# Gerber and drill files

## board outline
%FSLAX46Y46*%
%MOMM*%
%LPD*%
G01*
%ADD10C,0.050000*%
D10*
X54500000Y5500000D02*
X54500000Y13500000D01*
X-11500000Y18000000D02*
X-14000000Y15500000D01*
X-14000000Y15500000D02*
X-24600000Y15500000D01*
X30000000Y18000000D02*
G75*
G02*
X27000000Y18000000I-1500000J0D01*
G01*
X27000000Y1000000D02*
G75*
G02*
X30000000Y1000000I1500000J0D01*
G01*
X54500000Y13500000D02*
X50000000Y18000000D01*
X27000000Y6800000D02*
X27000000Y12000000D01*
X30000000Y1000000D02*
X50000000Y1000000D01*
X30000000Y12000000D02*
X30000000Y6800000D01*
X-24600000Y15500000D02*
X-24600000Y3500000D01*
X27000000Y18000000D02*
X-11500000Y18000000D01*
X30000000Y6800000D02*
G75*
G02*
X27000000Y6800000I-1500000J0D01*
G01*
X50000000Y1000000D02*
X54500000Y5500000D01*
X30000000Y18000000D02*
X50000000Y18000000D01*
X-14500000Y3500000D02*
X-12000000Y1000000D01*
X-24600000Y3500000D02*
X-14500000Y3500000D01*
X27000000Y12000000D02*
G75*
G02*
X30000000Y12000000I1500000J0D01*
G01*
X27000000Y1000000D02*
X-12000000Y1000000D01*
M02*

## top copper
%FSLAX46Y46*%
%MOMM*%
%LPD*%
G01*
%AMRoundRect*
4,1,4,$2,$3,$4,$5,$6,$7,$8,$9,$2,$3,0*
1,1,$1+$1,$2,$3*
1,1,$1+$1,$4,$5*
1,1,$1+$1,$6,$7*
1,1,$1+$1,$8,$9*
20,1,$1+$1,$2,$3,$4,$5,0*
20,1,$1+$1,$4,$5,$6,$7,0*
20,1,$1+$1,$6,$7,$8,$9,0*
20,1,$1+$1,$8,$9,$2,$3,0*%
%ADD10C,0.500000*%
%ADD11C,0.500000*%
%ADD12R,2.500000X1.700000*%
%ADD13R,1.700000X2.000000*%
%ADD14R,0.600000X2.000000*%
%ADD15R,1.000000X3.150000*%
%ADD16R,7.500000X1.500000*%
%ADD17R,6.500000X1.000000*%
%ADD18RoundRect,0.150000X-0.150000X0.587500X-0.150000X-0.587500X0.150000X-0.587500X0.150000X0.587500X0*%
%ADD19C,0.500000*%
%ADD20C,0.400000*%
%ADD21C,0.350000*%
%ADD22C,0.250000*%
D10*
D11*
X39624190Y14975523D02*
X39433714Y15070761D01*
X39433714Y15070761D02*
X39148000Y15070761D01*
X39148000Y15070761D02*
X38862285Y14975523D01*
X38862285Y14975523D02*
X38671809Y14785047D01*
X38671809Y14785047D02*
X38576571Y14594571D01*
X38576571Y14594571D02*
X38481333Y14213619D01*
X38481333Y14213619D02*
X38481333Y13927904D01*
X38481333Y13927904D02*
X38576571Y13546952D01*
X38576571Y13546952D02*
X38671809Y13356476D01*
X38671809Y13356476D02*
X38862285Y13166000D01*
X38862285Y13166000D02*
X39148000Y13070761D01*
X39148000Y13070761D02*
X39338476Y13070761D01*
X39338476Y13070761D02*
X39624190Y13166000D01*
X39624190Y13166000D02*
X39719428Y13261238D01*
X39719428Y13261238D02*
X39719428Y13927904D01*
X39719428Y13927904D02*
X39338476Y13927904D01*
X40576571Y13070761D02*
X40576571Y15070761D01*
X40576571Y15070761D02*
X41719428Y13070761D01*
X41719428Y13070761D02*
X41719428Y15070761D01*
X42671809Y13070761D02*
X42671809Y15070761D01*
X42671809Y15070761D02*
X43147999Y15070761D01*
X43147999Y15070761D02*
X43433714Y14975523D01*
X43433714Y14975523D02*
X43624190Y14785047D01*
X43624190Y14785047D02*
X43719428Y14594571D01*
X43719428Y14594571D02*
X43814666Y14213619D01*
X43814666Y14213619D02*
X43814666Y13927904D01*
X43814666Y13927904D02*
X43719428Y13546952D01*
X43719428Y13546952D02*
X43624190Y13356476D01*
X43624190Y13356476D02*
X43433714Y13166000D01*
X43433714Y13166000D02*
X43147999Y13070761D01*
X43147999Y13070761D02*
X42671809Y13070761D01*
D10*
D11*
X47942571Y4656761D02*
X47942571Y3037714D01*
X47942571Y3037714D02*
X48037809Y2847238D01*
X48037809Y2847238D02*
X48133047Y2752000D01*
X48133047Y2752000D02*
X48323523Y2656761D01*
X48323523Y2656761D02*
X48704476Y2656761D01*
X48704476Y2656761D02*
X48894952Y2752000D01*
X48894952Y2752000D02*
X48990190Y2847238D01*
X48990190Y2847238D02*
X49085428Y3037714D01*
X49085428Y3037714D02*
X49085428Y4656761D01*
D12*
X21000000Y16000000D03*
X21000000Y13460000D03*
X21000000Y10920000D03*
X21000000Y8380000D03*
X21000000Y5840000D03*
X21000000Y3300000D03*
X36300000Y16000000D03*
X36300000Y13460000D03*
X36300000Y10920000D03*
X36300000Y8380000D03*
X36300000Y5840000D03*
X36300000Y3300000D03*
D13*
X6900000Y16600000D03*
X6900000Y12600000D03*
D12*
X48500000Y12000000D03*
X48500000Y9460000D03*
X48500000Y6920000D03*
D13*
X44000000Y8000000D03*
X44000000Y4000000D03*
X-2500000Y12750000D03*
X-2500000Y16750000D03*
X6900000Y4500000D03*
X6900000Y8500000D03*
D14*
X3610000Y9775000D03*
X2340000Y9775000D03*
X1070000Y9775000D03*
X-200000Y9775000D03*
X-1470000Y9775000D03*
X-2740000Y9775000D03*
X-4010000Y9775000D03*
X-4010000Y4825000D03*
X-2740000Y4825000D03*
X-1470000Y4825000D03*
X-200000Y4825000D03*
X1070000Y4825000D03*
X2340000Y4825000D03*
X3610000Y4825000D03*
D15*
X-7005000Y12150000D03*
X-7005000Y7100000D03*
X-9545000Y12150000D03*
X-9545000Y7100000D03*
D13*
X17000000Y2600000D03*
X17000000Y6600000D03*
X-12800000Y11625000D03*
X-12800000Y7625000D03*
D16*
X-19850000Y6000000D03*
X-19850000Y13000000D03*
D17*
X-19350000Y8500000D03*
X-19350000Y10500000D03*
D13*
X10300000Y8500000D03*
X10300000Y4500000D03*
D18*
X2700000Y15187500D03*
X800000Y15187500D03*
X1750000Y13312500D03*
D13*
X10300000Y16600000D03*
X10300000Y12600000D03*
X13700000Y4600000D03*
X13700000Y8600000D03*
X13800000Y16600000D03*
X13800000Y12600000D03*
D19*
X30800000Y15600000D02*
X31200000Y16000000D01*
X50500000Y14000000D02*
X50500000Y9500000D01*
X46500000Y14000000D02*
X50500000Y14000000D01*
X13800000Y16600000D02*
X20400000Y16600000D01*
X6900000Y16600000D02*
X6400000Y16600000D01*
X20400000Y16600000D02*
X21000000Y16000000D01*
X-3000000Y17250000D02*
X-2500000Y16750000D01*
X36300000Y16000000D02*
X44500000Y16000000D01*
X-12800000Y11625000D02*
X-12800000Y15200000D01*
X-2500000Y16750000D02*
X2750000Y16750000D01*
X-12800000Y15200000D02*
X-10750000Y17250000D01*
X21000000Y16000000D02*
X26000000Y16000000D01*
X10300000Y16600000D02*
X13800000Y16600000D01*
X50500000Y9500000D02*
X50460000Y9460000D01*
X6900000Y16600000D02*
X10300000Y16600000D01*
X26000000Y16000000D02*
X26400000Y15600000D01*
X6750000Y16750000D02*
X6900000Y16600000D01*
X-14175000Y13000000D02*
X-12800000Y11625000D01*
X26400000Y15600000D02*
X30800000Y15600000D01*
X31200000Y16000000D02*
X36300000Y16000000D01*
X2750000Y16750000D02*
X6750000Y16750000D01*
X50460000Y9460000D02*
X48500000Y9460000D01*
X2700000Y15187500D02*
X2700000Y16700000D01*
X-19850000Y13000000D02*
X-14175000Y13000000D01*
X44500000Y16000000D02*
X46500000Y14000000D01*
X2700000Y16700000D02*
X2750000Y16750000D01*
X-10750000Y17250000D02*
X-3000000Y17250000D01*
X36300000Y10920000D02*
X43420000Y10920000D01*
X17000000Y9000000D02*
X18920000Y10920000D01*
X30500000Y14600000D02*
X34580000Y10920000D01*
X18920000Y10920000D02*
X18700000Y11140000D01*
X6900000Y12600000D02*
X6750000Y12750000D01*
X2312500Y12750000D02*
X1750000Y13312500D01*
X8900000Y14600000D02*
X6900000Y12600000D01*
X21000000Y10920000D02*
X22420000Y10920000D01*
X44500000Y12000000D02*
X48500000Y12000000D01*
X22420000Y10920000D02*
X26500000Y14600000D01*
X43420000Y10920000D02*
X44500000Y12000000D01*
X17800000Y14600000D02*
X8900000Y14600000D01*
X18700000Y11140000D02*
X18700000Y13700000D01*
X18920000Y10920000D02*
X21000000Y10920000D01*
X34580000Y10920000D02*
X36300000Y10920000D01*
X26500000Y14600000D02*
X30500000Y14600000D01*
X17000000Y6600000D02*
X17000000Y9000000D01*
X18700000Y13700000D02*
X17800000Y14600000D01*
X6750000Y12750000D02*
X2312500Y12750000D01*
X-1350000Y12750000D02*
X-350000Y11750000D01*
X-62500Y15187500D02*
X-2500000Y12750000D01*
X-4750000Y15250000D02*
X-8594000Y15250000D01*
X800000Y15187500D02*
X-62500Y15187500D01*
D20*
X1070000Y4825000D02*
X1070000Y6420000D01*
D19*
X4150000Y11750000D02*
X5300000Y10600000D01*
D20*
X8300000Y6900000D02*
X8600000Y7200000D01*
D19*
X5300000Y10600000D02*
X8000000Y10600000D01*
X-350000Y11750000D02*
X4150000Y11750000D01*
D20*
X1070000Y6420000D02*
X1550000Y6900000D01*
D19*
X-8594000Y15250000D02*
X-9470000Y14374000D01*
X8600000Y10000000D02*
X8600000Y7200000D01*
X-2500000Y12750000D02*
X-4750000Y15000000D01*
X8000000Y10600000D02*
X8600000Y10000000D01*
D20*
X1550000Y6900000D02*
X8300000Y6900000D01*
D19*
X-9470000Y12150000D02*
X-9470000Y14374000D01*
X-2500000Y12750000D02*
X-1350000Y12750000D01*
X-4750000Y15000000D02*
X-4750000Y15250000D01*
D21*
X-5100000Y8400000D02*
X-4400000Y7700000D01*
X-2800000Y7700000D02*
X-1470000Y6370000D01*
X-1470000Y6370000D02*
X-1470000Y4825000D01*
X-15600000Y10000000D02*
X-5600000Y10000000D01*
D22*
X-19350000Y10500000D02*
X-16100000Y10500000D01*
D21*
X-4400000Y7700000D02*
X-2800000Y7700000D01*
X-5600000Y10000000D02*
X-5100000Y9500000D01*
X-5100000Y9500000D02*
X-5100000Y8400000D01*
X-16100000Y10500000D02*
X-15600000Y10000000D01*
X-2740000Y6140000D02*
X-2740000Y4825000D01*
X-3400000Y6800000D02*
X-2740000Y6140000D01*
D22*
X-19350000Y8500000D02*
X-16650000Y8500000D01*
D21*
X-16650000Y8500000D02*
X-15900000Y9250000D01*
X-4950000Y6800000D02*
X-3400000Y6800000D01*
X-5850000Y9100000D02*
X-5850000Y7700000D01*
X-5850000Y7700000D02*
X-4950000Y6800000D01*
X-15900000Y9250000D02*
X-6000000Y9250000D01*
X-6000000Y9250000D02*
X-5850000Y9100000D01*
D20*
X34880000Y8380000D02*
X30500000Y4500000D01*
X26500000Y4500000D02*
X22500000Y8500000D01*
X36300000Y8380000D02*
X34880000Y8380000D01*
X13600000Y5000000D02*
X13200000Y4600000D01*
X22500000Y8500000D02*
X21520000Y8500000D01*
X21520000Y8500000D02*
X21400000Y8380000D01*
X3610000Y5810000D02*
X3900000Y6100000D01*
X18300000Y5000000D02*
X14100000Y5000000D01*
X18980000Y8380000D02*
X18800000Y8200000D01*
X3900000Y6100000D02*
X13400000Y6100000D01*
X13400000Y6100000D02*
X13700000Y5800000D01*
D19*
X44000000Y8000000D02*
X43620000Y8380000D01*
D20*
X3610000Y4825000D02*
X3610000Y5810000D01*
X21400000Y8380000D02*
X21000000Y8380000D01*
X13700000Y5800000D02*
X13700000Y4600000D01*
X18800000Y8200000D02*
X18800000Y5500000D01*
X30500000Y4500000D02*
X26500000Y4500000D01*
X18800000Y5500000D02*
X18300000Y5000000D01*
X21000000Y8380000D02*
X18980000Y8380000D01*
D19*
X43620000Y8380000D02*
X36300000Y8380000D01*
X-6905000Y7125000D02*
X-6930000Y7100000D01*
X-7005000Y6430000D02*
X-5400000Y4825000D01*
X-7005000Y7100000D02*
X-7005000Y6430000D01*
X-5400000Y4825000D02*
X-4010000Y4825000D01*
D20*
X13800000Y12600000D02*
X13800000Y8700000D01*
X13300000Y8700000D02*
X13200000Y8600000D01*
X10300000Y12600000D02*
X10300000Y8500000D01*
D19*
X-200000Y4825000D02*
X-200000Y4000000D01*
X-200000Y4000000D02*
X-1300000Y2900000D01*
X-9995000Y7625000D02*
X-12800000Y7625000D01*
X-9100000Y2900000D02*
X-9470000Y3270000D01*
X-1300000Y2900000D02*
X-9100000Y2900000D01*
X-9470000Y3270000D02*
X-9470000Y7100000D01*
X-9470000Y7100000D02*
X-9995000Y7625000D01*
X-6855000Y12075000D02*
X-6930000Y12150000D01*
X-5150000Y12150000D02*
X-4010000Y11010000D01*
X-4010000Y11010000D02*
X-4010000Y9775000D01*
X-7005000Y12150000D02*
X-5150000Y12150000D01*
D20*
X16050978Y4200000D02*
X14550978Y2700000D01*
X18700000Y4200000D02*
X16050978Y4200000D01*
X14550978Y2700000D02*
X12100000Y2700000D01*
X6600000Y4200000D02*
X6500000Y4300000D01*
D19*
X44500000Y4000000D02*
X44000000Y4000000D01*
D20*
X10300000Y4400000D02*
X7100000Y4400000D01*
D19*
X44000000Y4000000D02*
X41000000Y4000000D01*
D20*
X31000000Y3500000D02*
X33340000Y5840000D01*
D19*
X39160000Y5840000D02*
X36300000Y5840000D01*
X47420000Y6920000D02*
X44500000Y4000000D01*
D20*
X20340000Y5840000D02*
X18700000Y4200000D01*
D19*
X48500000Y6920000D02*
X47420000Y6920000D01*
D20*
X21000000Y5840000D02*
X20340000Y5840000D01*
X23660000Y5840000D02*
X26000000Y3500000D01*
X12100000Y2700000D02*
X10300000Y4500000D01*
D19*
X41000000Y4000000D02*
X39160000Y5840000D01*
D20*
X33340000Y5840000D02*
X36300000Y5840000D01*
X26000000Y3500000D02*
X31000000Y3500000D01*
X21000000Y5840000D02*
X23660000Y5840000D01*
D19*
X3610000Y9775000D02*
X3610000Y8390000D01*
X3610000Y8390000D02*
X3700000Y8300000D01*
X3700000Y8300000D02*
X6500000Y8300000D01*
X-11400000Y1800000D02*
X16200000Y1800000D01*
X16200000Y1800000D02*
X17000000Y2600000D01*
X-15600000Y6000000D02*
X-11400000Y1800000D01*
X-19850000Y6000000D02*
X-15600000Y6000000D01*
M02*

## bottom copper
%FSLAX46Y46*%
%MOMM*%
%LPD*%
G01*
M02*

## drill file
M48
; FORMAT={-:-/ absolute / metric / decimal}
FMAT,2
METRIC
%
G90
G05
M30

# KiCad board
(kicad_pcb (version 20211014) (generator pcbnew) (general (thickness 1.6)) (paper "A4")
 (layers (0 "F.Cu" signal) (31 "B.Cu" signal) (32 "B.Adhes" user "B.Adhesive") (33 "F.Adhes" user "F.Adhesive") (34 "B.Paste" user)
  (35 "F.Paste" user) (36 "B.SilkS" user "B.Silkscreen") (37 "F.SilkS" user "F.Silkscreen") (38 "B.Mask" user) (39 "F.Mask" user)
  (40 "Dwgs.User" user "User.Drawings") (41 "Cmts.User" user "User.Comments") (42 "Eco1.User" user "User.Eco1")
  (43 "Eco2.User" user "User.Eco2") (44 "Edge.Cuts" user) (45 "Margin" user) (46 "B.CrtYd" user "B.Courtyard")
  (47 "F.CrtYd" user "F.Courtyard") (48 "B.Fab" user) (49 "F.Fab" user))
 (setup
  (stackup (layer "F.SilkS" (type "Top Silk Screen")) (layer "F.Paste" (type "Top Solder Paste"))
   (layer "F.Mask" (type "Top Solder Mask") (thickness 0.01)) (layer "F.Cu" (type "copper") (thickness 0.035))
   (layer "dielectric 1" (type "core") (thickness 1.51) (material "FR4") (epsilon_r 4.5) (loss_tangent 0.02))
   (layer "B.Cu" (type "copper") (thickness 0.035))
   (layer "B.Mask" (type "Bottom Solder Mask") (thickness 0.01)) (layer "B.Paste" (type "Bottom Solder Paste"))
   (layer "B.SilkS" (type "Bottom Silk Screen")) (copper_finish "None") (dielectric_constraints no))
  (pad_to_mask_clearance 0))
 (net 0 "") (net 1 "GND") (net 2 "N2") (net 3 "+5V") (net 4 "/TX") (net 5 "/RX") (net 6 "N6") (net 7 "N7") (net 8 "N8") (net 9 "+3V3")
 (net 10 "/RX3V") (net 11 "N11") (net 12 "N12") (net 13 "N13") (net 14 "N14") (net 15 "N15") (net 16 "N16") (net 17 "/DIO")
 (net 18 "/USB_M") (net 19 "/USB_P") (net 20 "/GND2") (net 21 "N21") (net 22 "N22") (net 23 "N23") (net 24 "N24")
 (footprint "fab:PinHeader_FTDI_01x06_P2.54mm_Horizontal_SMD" (layer "F.Cu") (at 21 -16)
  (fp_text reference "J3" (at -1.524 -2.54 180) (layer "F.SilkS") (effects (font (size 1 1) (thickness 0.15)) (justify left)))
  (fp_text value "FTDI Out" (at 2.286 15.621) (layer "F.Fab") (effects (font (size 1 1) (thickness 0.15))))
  (pad "1" smd rect locked (at 0 0) (size 2.5 1.7) (layers "F.Cu" "F.Paste" "F.Mask") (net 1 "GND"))
  (pad "2" smd rect locked (at 0 2.54) (size 2.5 1.7) (layers "F.Cu" "F.Paste" "F.Mask") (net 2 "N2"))
  (pad "3" smd rect locked (at 0 5.08) (size 2.5 1.7) (layers "F.Cu" "F.Paste" "F.Mask") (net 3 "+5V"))
  (pad "4" smd rect locked (at 0 7.62) (size 2.5 1.7) (layers "F.Cu" "F.Paste" "F.Mask") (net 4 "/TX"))
  (pad "5" smd rect locked (at 0 10.16) (size 2.5 1.7) (layers "F.Cu" "F.Paste" "F.Mask") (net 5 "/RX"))
  (pad "6" smd rect locked (at 0 12.7) (size 2.5 1.7) (layers "F.Cu" "F.Paste" "F.Mask") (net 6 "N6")))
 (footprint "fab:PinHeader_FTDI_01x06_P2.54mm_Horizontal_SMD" (layer "F.Cu") (at 36.3 -16)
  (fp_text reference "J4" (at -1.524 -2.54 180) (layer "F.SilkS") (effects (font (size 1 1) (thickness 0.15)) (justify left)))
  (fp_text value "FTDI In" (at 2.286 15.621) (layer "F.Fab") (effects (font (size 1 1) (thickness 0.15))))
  (pad "1" smd rect locked (at 0 0) (size 2.5 1.7) (layers "F.Cu" "F.Paste" "F.Mask") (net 1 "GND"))
  (pad "2" smd rect locked (at 0 2.54) (size 2.5 1.7) (layers "F.Cu" "F.Paste" "F.Mask") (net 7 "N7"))
  (pad "3" smd rect locked (at 0 5.08) (size 2.5 1.7) (layers "F.Cu" "F.Paste" "F.Mask") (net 3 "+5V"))
  (pad "4" smd rect locked (at 0 7.62) (size 2.5 1.7) (layers "F.Cu" "F.Paste" "F.Mask") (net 4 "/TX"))
  (pad "5" smd rect locked (at 0 10.16) (size 2.5 1.7) (layers "F.Cu" "F.Paste" "F.Mask") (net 5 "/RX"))
  (pad "6" smd rect locked (at 0 12.7) (size 2.5 1.7) (layers "F.Cu" "F.Paste" "F.Mask") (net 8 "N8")))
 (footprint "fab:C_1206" (layer "F.Cu") (at 6.9 -14.6 -90)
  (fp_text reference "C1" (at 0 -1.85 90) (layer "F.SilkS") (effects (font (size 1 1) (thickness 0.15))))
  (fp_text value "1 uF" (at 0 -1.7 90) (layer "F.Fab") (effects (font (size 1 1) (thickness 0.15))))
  (pad "1" smd rect locked (at -2 0 270) (size 2 1.7) (layers "F.Cu" "F.Paste" "F.Mask") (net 1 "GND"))
  (pad "2" smd rect locked (at 2 0 270) (size 2 1.7) (layers "F.Cu" "F.Paste" "F.Mask") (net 3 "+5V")))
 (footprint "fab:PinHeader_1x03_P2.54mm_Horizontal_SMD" (layer "F.Cu") (at 48.5 -12)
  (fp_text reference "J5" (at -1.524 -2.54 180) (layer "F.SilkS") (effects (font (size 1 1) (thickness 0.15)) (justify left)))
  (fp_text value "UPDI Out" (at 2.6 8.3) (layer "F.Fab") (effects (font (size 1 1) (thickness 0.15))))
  (pad "1" smd rect locked (at 0 0) (size 2.5 1.7) (layers "F.Cu" "F.Paste" "F.Mask") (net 3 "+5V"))
  (pad "2" smd rect locked (at 0 2.54) (size 2.5 1.7) (layers "F.Cu" "F.Paste" "F.Mask") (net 1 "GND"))
  (pad "3" smd rect locked (at 0 5.08) (size 2.5 1.7) (layers "F.Cu" "F.Paste" "F.Mask") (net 5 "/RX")))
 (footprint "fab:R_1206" (layer "F.Cu") (at 44 -6 -90)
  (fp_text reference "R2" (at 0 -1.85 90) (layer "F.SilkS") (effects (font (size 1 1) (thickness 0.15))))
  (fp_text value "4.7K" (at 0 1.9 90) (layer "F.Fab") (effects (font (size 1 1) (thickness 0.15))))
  (pad "1" smd rect locked (at -2 0 270) (size 2 1.7) (layers "F.Cu" "F.Paste" "F.Mask") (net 4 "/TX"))
  (pad "2" smd rect locked (at 2 0 270) (size 2 1.7) (layers "F.Cu" "F.Paste" "F.Mask") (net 5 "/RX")))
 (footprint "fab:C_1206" (layer "F.Cu") (at -2.5 -14.75 90)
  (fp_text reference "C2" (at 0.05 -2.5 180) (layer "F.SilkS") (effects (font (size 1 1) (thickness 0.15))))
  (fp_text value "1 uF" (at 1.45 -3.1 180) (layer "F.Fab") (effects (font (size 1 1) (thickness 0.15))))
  (pad "1" smd rect locked (at -2 0 90) (size 2 1.7) (layers "F.Cu" "F.Paste" "F.Mask") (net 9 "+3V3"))
  (pad "2" smd rect locked (at 2 0 90) (size 2 1.7) (layers "F.Cu" "F.Paste" "F.Mask") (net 1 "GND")))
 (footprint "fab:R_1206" (layer "F.Cu") (at 6.9 -6.5 90)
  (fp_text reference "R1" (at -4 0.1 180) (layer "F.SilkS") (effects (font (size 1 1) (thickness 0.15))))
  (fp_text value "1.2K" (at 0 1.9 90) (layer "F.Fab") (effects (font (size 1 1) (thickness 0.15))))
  (pad "1" smd rect locked (at -2 0 90) (size 2 1.7) (layers "F.Cu" "F.Paste" "F.Mask") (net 5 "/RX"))
  (pad "2" smd rect locked (at 2 0 90) (size 2 1.7) (layers "F.Cu" "F.Paste" "F.Mask") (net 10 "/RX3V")))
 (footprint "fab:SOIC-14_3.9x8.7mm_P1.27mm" (layer "F.Cu") (at -0.2 -7.3 -90)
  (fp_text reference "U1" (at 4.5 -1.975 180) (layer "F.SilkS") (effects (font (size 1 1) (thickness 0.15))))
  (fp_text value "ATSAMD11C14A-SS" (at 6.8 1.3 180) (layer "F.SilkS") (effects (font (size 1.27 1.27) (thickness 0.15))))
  (pad "1" smd rect locked (at -2.475 -3.81 270) (size 2 0.6) (layers "F.Cu" "F.Paste" "F.Mask") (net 10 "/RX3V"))
  (pad "2" smd rect locked (at -2.475 -2.54 270) (size 2 0.6) (layers "F.Cu" "F.Paste" "F.Mask") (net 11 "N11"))
  (pad "3" smd rect locked (at -2.475 -1.27 270) (size 2 0.6) (layers "F.Cu" "F.Paste" "F.Mask") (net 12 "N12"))
  (pad "4" smd rect locked (at -2.475 0 270) (size 2 0.6) (layers "F.Cu" "F.Paste" "F.Mask") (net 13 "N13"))
  (pad "5" smd rect locked (at -2.475 1.27 270) (size 2 0.6) (layers "F.Cu" "F.Paste" "F.Mask") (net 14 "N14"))
  (pad "6" smd rect locked (at -2.475 2.54 270) (size 2 0.6) (layers "F.Cu" "F.Paste" "F.Mask") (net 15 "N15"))
  (pad "7" smd rect locked (at -2.475 3.81 270) (size 2 0.6) (layers "F.Cu" "F.Paste" "F.Mask") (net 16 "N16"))
  (pad "8" smd rect locked (at 2.475 3.81 270) (size 2 0.6) (layers "F.Cu" "F.Paste" "F.Mask") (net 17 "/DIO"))
  (pad "9" smd rect locked (at 2.475 2.54 270) (size 2 0.6) (layers "F.Cu" "F.Paste" "F.Mask") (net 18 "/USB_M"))
  (pad "10" smd rect locked (at 2.475 1.27 270) (size 2 0.6) (layers "F.Cu" "F.Paste" "F.Mask") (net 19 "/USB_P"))
  (pad "11" smd rect locked (at 2.475 0 270) (size 2 0.6) (layers "F.Cu" "F.Paste" "F.Mask") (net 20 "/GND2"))
  (pad "12" smd rect locked (at 2.475 -1.27 270) (size 2 0.6) (layers "F.Cu" "F.Paste" "F.Mask") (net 9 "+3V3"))
  (pad "13" smd rect locked (at 2.475 -2.54 270) (size 2 0.6) (layers "F.Cu" "F.Paste" "F.Mask") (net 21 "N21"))
  (pad "14" smd rect locked (at 2.475 -3.81 270) (size 2 0.6) (layers "F.Cu" "F.Paste" "F.Mask") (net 4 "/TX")))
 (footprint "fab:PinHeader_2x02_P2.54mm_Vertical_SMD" (layer "F.Cu") (at -8.275 -9.625 -90)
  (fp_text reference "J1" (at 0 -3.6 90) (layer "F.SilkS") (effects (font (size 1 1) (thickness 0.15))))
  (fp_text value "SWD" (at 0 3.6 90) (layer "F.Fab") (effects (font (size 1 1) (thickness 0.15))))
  (pad "1" smd rect locked (at -2.525 -1.27 270) (size 3.15 1) (layers "F.Cu" "F.Paste" "F.Mask") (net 16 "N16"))
  (pad "2" smd rect locked (at 2.525 -1.27 270) (size 3.15 1) (layers "F.Cu" "F.Paste" "F.Mask") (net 17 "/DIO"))
  (pad "3" smd rect locked (at -2.525 1.27 270) (size 3.15 1) (layers "F.Cu" "F.Paste" "F.Mask") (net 9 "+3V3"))
  (pad "4" smd rect locked (at 2.525 1.27 270) (size 3.15 1) (layers "F.Cu" "F.Paste" "F.Mask") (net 20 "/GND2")))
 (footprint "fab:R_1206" (layer "F.Cu") (at 17 -4.6 90)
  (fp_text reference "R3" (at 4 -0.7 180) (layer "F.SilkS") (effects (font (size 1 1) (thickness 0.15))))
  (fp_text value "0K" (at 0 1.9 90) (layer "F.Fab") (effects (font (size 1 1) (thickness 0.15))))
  (pad "1" smd rect locked (at -2 0 90) (size 2 1.7) (layers "F.Cu" "F.Paste" "F.Mask") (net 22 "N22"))
  (pad "2" smd rect locked (at 2 0 90) (size 2 1.7) (layers "F.Cu" "F.Paste" "F.Mask") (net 3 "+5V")))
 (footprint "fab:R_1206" (layer "F.Cu") (at -12.8 -9.625 -90)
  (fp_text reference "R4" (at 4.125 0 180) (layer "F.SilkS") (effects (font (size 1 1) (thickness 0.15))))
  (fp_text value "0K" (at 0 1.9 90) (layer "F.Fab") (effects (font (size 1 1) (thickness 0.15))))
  (pad "1" smd rect locked (at -2 0 270) (size 2 1.7) (layers "F.Cu" "F.Paste" "F.Mask") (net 1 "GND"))
  (pad "2" smd rect locked (at 2 0 270) (size 2 1.7) (layers "F.Cu" "F.Paste" "F.Mask") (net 20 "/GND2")))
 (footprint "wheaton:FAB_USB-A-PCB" (layer "F.Cu") (at -19.65 -9.5)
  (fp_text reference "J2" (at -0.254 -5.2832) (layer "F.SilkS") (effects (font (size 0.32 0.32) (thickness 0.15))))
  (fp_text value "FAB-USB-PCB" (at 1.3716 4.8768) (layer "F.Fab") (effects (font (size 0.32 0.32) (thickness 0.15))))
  (pad "5V" smd rect locked (at -0.2 3.5) (size 7.5 1.5) (layers "F.Cu" "F.Paste" "F.Mask") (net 22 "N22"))
  (pad "GND" smd rect locked (at -0.2 -3.5) (size 7.5 1.5) (layers "F.Cu" "F.Paste" "F.Mask") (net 1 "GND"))
  (pad "USB_M" smd rect locked (at 0.3 1) (size 6.5 1) (layers "F.Cu" "F.Paste" "F.Mask") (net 18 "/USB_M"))
  (pad "USB_P" smd rect locked (at 0.3 -1) (size 6.5 1) (layers "F.Cu" "F.Paste" "F.Mask") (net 19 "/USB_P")))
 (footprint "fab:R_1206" (layer "F.Cu") (at 10.3 -6.5 -90)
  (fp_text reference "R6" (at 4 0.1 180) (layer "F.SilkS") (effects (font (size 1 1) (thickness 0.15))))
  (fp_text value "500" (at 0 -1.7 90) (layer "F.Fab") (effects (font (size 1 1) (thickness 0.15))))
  (pad "1" smd rect locked (at -2 0 270) (size 2 1.7) (layers "F.Cu" "F.Paste" "F.Mask") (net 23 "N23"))
  (pad "2" smd rect locked (at 2 0 270) (size 2 1.7) (layers "F.Cu" "F.Paste" "F.Mask") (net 5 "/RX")))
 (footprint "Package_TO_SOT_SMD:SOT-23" (layer "F.Cu") (at 1.75 -14.25 -90)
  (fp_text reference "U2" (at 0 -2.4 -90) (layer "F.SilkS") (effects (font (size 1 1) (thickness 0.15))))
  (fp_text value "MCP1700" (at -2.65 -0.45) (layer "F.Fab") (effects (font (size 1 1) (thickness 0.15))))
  (pad "1" smd roundrect (at -0.9375 -0.95 270) (size 1.475 0.6) (layers "F.Cu" "F.Paste" "F.Mask") (roundrect_rratio 0.25) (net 1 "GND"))
  (pad "2" smd roundrect (at -0.9375 0.95 270) (size 1.475 0.6) (layers "F.Cu" "F.Paste" "F.Mask") (roundrect_rratio 0.25) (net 9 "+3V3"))
  (pad "3" smd roundrect (at 0.9375 0 270) (size 1.475 0.6) (layers "F.Cu" "F.Paste" "F.Mask") (roundrect_rratio 0.25) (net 3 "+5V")))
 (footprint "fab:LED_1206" (layer "F.Cu") (at 10.3 -14.6 -90)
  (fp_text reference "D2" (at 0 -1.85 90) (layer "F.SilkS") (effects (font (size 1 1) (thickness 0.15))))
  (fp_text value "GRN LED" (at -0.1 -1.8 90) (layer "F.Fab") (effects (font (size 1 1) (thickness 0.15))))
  (pad "1" smd rect locked (at -2 0 270) (size 2 1.7) (layers "F.Cu" "F.Paste" "F.Mask") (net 1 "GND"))
  (pad "2" smd rect locked (at 2 0 270) (size 2 1.7) (layers "F.Cu" "F.Paste" "F.Mask") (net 23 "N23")))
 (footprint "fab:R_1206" (layer "F.Cu") (at 13.7 -6.6 90)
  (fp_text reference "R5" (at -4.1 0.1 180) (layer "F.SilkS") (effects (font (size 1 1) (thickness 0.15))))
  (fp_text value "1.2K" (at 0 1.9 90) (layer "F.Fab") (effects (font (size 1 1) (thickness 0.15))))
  (pad "1" smd rect locked (at -2 0 90) (size 2 1.7) (layers "F.Cu" "F.Paste" "F.Mask") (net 4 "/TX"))
  (pad "2" smd rect locked (at 2 0 90) (size 2 1.7) (layers "F.Cu" "F.Paste" "F.Mask") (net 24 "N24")))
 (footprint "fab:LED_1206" (layer "F.Cu") (at 13.8 -14.6 -90)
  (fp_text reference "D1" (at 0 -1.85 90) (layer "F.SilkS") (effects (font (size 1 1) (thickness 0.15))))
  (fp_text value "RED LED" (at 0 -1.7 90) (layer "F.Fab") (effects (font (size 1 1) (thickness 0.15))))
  (pad "1" smd rect locked (at -2 0 270) (size 2 1.7) (layers "F.Cu" "F.Paste" "F.Mask") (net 1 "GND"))
  (pad "2" smd rect locked (at 2 0 270) (size 2 1.7) (layers "F.Cu" "F.Paste" "F.Mask") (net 24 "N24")))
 (gr_line (start 54.5 -5.5) (end 54.5 -13.5) (layer "Edge.Cuts") (width 0.05))
 (gr_line (start -11.5 -18) (end -14 -15.5) (layer "Edge.Cuts") (width 0.05))
 (gr_line (start -14 -15.5) (end -24.6 -15.5) (layer "Edge.Cuts") (width 0.05))
 (gr_arc (start 30 -18) (mid 28.5 -16.5) (end 27 -18) (layer "Edge.Cuts") (width 0.05))
 (gr_arc (start 27 -1) (mid 28.5 -2.5) (end 30 -1) (layer "Edge.Cuts") (width 0.05))
 (gr_line (start 54.5 -13.5) (end 50 -18) (layer "Edge.Cuts") (width 0.05))
 (gr_line (start 27 -6.8) (end 27 -12) (layer "Edge.Cuts") (width 0.05))
 (gr_line (start 30 -1) (end 50 -1) (layer "Edge.Cuts") (width 0.05))
 (gr_line (start 30 -12) (end 30 -6.8) (layer "Edge.Cuts") (width 0.05))
 (gr_line (start -24.6 -15.5) (end -24.6 -3.5) (layer "Edge.Cuts") (width 0.05))
 (gr_line (start 27 -18) (end -11.5 -18) (layer "Edge.Cuts") (width 0.05))
 (gr_arc (start 30 -6.8) (mid 28.5 -5.3) (end 27 -6.8) (layer "Edge.Cuts") (width 0.05))
 (gr_line (start 50 -1) (end 54.5 -5.5) (layer "Edge.Cuts") (width 0.05))
 (gr_line (start 30 -18) (end 50 -18) (layer "Edge.Cuts") (width 0.05))
 (gr_line (start -14.5 -3.5) (end -12 -1) (layer "Edge.Cuts") (width 0.05))
 (gr_line (start -24.6 -3.5) (end -14.5 -3.5) (layer "Edge.Cuts") (width 0.05))
 (gr_arc (start 27 -12) (mid 28.5 -13.5) (end 30 -12) (layer "Edge.Cuts") (width 0.05))
 (gr_line (start 27 -1) (end -12 -1) (layer "Edge.Cuts") (width 0.05))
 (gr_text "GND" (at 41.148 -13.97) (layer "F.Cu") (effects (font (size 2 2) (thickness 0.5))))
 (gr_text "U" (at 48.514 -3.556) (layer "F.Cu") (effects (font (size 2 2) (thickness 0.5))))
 (segment (start 30.8 -15.6) (end 31.2 -16) (width 0.5) (layer "F.Cu") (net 1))
 (segment (start 50.5 -14) (end 50.5 -9.5) (width 0.5) (layer "F.Cu") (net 1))
 (segment (start 46.5 -14) (end 50.5 -14) (width 0.5) (layer "F.Cu") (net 1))
 (segment (start 13.8 -16.6) (end 20.4 -16.6) (width 0.5) (layer "F.Cu") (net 1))
 (segment (start 6.9 -16.6) (end 6.4 -16.6) (width 0.5) (layer "F.Cu") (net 1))
 (segment (start 20.4 -16.6) (end 21 -16) (width 0.5) (layer "F.Cu") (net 1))
 (segment (start -3 -17.25) (end -2.5 -16.75) (width 0.5) (layer "F.Cu") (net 1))
 (segment (start 36.3 -16) (end 44.5 -16) (width 0.5) (layer "F.Cu") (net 1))
 (segment (start -12.8 -11.625) (end -12.8 -15.2) (width 0.5) (layer "F.Cu") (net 1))
 (segment (start -2.5 -16.75) (end 2.75 -16.75) (width 0.5) (layer "F.Cu") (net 1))
 (segment (start -12.8 -15.2) (end -10.75 -17.25) (width 0.5) (layer "F.Cu") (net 1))
 (segment (start 21 -16) (end 26 -16) (width 0.5) (layer "F.Cu") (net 1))
 (segment (start 10.3 -16.6) (end 13.8 -16.6) (width 0.5) (layer "F.Cu") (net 1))
 (segment (start 50.5 -9.5) (end 50.46 -9.46) (width 0.5) (layer "F.Cu") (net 1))
 (segment (start 6.9 -16.6) (end 10.3 -16.6) (width 0.5) (layer "F.Cu") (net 1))
 (segment (start 26 -16) (end 26.4 -15.6) (width 0.5) (layer "F.Cu") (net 1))
 (segment (start 6.75 -16.75) (end 6.9 -16.6) (width 0.5) (layer "F.Cu") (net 1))
 (segment (start -14.175 -13) (end -12.8 -11.625) (width 0.5) (layer "F.Cu") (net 1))
 (segment (start 26.4 -15.6) (end 30.8 -15.6) (width 0.5) (layer "F.Cu") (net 1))
 (segment (start 31.2 -16) (end 36.3 -16) (width 0.5) (layer "F.Cu") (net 1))
 (segment (start 2.75 -16.75) (end 6.75 -16.75) (width 0.5) (layer "F.Cu") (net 1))
 (segment (start 50.46 -9.46) (end 48.5 -9.46) (width 0.5) (layer "F.Cu") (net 1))
 (segment (start 2.7 -15.1875) (end 2.7 -16.7) (width 0.5) (layer "F.Cu") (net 1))
 (segment (start -19.85 -13) (end -14.175 -13) (width 0.5) (layer "F.Cu") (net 1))
 (segment (start 44.5 -16) (end 46.5 -14) (width 0.5) (layer "F.Cu") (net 1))
 (segment (start 2.7 -16.7) (end 2.75 -16.75) (width 0.5) (layer "F.Cu") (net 1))
 (segment (start -10.75 -17.25) (end -3 -17.25) (width 0.5) (layer "F.Cu") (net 1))
 (segment (start 36.3 -10.92) (end 43.42 -10.92) (width 0.5) (layer "F.Cu") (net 3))
 (segment (start 17 -9) (end 18.92 -10.92) (width 0.5) (layer "F.Cu") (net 3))
 (segment (start 30.5 -14.6) (end 34.58 -10.92) (width 0.5) (layer "F.Cu") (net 3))
 (segment (start 18.92 -10.92) (end 18.7 -11.14) (width 0.5) (layer "F.Cu") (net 3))
 (segment (start 6.9 -12.6) (end 6.75 -12.75) (width 0.5) (layer "F.Cu") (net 3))
 (segment (start 2.3125 -12.75) (end 1.75 -13.3125) (width 0.5) (layer "F.Cu") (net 3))
 (segment (start 8.9 -14.6) (end 6.9 -12.6) (width 0.5) (layer "F.Cu") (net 3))
 (segment (start 21 -10.92) (end 22.42 -10.92) (width 0.5) (layer "F.Cu") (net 3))
 (segment (start 44.5 -12) (end 48.5 -12) (width 0.5) (layer "F.Cu") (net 3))
 (segment (start 22.42 -10.92) (end 26.5 -14.6) (width 0.5) (layer "F.Cu") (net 3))
 (segment (start 43.42 -10.92) (end 44.5 -12) (width 0.5) (layer "F.Cu") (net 3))
 (segment (start 17.8 -14.6) (end 8.9 -14.6) (width 0.5) (layer "F.Cu") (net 3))
 (segment (start 18.7 -11.14) (end 18.7 -13.7) (width 0.5) (layer "F.Cu") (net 3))
 (segment (start 18.92 -10.92) (end 21 -10.92) (width 0.5) (layer "F.Cu") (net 3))
 (segment (start 34.58 -10.92) (end 36.3 -10.92) (width 0.5) (layer "F.Cu") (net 3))
 (segment (start 26.5 -14.6) (end 30.5 -14.6) (width 0.5) (layer "F.Cu") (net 3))
 (segment (start 17 -6.6) (end 17 -9) (width 0.5) (layer "F.Cu") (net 3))
 (segment (start 18.7 -13.7) (end 17.8 -14.6) (width 0.5) (layer "F.Cu") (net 3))
 (segment (start 6.75 -12.75) (end 2.3125 -12.75) (width 0.5) (layer "F.Cu") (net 3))
 (segment (start -1.35 -12.75) (end -0.35 -11.75) (width 0.5) (layer "F.Cu") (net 9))
 (segment (start -0.0625 -15.1875) (end -2.5 -12.75) (width 0.5) (layer "F.Cu") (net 9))
 (segment (start -4.75 -15.25) (end -8.594 -15.25) (width 0.5) (layer "F.Cu") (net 9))
 (segment (start 0.8 -15.1875) (end -0.0625 -15.1875) (width 0.5) (layer "F.Cu") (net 9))
 (segment (start 1.07 -4.825) (end 1.07 -6.42) (width 0.4) (layer "F.Cu") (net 9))
 (segment (start 4.15 -11.75) (end 5.3 -10.6) (width 0.5) (layer "F.Cu") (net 9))
 (segment (start 8.3 -6.9) (end 8.6 -7.2) (width 0.4) (layer "F.Cu") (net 9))
 (segment (start 5.3 -10.6) (end 8 -10.6) (width 0.5) (layer "F.Cu") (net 9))
 (segment (start -0.35 -11.75) (end 4.15 -11.75) (width 0.5) (layer "F.Cu") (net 9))
 (segment (start 1.07 -6.42) (end 1.55 -6.9) (width 0.4) (layer "F.Cu") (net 9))
 (segment (start -8.594 -15.25) (end -9.47 -14.374) (width 0.5) (layer "F.Cu") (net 9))
 (segment (start 8.6 -10) (end 8.6 -7.2) (width 0.5) (layer "F.Cu") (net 9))
 (segment (start -2.5 -12.75) (end -4.75 -15) (width 0.5) (layer "F.Cu") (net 9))
 (segment (start 8 -10.6) (end 8.6 -10) (width 0.5) (layer "F.Cu") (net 9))
 (segment (start 1.55 -6.9) (end 8.3 -6.9) (width 0.4) (layer "F.Cu") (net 9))
 (segment (start -9.47 -12.15) (end -9.47 -14.374) (width 0.5) (layer "F.Cu") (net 9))
 (segment (start -2.5 -12.75) (end -1.35 -12.75) (width 0.5) (layer "F.Cu") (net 9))
 (segment (start -4.75 -15) (end -4.75 -15.25) (width 0.5) (layer "F.Cu") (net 9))
 (segment (start -5.1 -8.4) (end -4.4 -7.7) (width 0.35) (layer "F.Cu") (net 19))
 (segment (start -2.8 -7.7) (end -1.47 -6.37) (width 0.35) (layer "F.Cu") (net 19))
 (segment (start -1.47 -6.37) (end -1.47 -4.825) (width 0.35) (layer "F.Cu") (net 19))
 (segment (start -15.6 -10) (end -5.6 -10) (width 0.35) (layer "F.Cu") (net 19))
 (segment (start -19.35 -10.5) (end -16.1 -10.5) (width 0.25) (layer "F.Cu") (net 19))
 (segment (start -4.4 -7.7) (end -2.8 -7.7) (width 0.35) (layer "F.Cu") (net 19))
 (segment (start -5.6 -10) (end -5.1 -9.5) (width 0.35) (layer "F.Cu") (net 19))
 (segment (start -5.1 -9.5) (end -5.1 -8.4) (width 0.35) (layer "F.Cu") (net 19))
 (segment (start -16.1 -10.5) (end -15.6 -10) (width 0.35) (layer "F.Cu") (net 19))
 (segment (start -2.74 -6.14) (end -2.74 -4.825) (width 0.35) (layer "F.Cu") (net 18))
 (segment (start -3.4 -6.8) (end -2.74 -6.14) (width 0.35) (layer "F.Cu") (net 18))
 (segment (start -19.35 -8.5) (end -16.65 -8.5) (width 0.25) (layer "F.Cu") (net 18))
 (segment (start -16.65 -8.5) (end -15.9 -9.25) (width 0.35) (layer "F.Cu") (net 18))
 (segment (start -4.95 -6.8) (end -3.4 -6.8) (width 0.35) (layer "F.Cu") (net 18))
 (segment (start -5.85 -9.1) (end -5.85 -7.7) (width 0.35) (layer "F.Cu") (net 18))
 (segment (start -5.85 -7.7) (end -4.95 -6.8) (width 0.35) (layer "F.Cu") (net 18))
 (segment (start -15.9 -9.25) (end -6 -9.25) (width 0.35) (layer "F.Cu") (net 18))
 (segment (start -6 -9.25) (end -5.85 -9.1) (width 0.35) (layer "F.Cu") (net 18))
 (segment (start 34.88 -8.38) (end 30.5 -4.5) (width 0.4) (layer "F.Cu") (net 4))
 (segment (start 26.5 -4.5) (end 22.5 -8.5) (width 0.4) (layer "F.Cu") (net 4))
 (segment (start 36.3 -8.38) (end 34.88 -8.38) (width 0.4) (layer "F.Cu") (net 4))
 (segment (start 13.6 -5) (end 13.2 -4.6) (width 0.4) (layer "F.Cu") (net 4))
 (segment (start 22.5 -8.5) (end 21.52 -8.5) (width 0.4) (layer "F.Cu") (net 4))
 (segment (start 21.52 -8.5) (end 21.4 -8.38) (width 0.4) (layer "F.Cu") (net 4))
 (segment (start 3.61 -5.81) (end 3.9 -6.1) (width 0.4) (layer "F.Cu") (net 4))
 (segment (start 18.3 -5) (end 14.1 -5) (width 0.4) (layer "F.Cu") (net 4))
 (segment (start 18.98 -8.38) (end 18.8 -8.2) (width 0.4) (layer "F.Cu") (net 4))
 (segment (start 3.9 -6.1) (end 13.4 -6.1) (width 0.4) (layer "F.Cu") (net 4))
 (segment (start 13.4 -6.1) (end 13.7 -5.8) (width 0.4) (layer "F.Cu") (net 4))
 (segment (start 44 -8) (end 43.62 -8.38) (width 0.5) (layer "F.Cu") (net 4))
 (segment (start 3.61 -4.825) (end 3.61 -5.81) (width 0.4) (layer "F.Cu") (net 4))
 (segment (start 21.4 -8.38) (end 21 -8.38) (width 0.4) (layer "F.Cu") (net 4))
 (segment (start 13.7 -5.8) (end 13.7 -4.6) (width 0.4) (layer "F.Cu") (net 4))
 (segment (start 18.8 -8.2) (end 18.8 -5.5) (width 0.4) (layer "F.Cu") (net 4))
 (segment (start 30.5 -4.5) (end 26.5 -4.5) (width 0.4) (layer "F.Cu") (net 4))
 (segment (start 18.8 -5.5) (end 18.3 -5) (width 0.4) (layer "F.Cu") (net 4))
 (segment (start 21 -8.38) (end 18.98 -8.38) (width 0.4) (layer "F.Cu") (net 4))
 (segment (start 43.62 -8.38) (end 36.3 -8.38) (width 0.5) (layer "F.Cu") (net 4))
 (segment (start -6.905 -7.125) (end -6.93 -7.1) (width 0.5) (layer "F.Cu") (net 17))
 (segment (start -7.005 -6.43) (end -5.4 -4.825) (width 0.5) (layer "F.Cu") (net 17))
 (segment (start -7.005 -7.1) (end -7.005 -6.43) (width 0.5) (layer "F.Cu") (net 17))
 (segment (start -5.4 -4.825) (end -4.01 -4.825) (width 0.5) (layer "F.Cu") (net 17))
 (segment (start 13.8 -12.6) (end 13.8 -8.7) (width 0.4) (layer "F.Cu") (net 24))
 (segment (start 13.3 -8.7) (end 13.2 -8.6) (width 0.4) (layer "F.Cu") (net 24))
 (segment (start 10.3 -12.6) (end 10.3 -8.5) (width 0.4) (layer "F.Cu") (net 23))
 (segment (start -0.2 -4.825) (end -0.2 -4) (width 0.5) (layer "F.Cu") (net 20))
 (segment (start -0.2 -4) (end -1.3 -2.9) (width 0.5) (layer "F.Cu") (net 20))
 (segment (start -9.995 -7.625) (end -12.8 -7.625) (width 0.5) (layer "F.Cu") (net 20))
 (segment (start -9.1 -2.9) (end -9.47 -3.27) (width 0.5) (layer "F.Cu") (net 20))
 (segment (start -1.3 -2.9) (end -9.1 -2.9) (width 0.5) (layer "F.Cu") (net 20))
 (segment (start -9.47 -3.27) (end -9.47 -7.1) (width 0.5) (layer "F.Cu") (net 20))
 (segment (start -9.47 -7.1) (end -9.995 -7.625) (width 0.5) (layer "F.Cu") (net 20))
 (segment (start -6.855 -12.075) (end -6.93 -12.15) (width 0.5) (layer "F.Cu") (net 16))
 (segment (start -5.15 -12.15) (end -4.01 -11.01) (width 0.5) (layer "F.Cu") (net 16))
 (segment (start -4.01 -11.01) (end -4.01 -9.775) (width 0.5) (layer "F.Cu") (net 16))
 (segment (start -7.005 -12.15) (end -5.15 -12.15) (width 0.5) (layer "F.Cu") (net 16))
 (segment (start 16.050978 -4.2) (end 14.550978 -2.7) (width 0.4) (layer "F.Cu") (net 5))
 (segment (start 18.7 -4.2) (end 16.050978 -4.2) (width 0.4) (layer "F.Cu") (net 5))
 (segment (start 14.550978 -2.7) (end 12.1 -2.7) (width 0.4) (layer "F.Cu") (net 5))
 (segment (start 6.6 -4.2) (end 6.5 -4.3) (width 0.4) (layer "F.Cu") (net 5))
 (segment (start 44.5 -4) (end 44 -4) (width 0.5) (layer "F.Cu") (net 5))
 (segment (start 10.3 -4.4) (end 7.1 -4.4) (width 0.4) (layer "F.Cu") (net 5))
 (segment (start 44 -4) (end 41 -4) (width 0.5) (layer "F.Cu") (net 5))
 (segment (start 31 -3.5) (end 33.34 -5.84) (width 0.4) (layer "F.Cu") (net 5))
 (segment (start 39.16 -5.84) (end 36.3 -5.84) (width 0.5) (layer "F.Cu") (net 5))
 (segment (start 47.42 -6.92) (end 44.5 -4) (width 0.5) (layer "F.Cu") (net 5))
 (segment (start 20.34 -5.84) (end 18.7 -4.2) (width 0.4) (layer "F.Cu") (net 5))
 (segment (start 48.5 -6.92) (end 47.42 -6.92) (width 0.5) (layer "F.Cu") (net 5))
 (segment (start 21 -5.84) (end 20.34 -5.84) (width 0.4) (layer "F.Cu") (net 5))
 (segment (start 23.66 -5.84) (end 26 -3.5) (width 0.4) (layer "F.Cu") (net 5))
 (segment (start 12.1 -2.7) (end 10.3 -4.5) (width 0.4) (layer "F.Cu") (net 5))
 (segment (start 41 -4) (end 39.16 -5.84) (width 0.5) (layer "F.Cu") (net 5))
 (segment (start 33.34 -5.84) (end 36.3 -5.84) (width 0.4) (layer "F.Cu") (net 5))
 (segment (start 26 -3.5) (end 31 -3.5) (width 0.4) (layer "F.Cu") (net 5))
 (segment (start 21 -5.84) (end 23.66 -5.84) (width 0.4) (layer "F.Cu") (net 5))
 (segment (start 3.61 -9.775) (end 3.61 -8.39) (width 0.5) (layer "F.Cu") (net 10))
 (segment (start 3.61 -8.39) (end 3.7 -8.3) (width 0.5) (layer "F.Cu") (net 10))
 (segment (start 3.7 -8.3) (end 6.5 -8.3) (width 0.5) (layer "F.Cu") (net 10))
 (segment (start -11.4 -1.8) (end 16.2 -1.8) (width 0.5) (layer "F.Cu") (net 22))
 (segment (start 16.2 -1.8) (end 17 -2.6) (width 0.5) (layer "F.Cu") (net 22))
 (segment (start -15.6 -6) (end -11.4 -1.8) (width 0.5) (layer "F.Cu") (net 22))
 (segment (start -19.85 -6) (end -15.6 -6) (width 0.5) (layer "F.Cu") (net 22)))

